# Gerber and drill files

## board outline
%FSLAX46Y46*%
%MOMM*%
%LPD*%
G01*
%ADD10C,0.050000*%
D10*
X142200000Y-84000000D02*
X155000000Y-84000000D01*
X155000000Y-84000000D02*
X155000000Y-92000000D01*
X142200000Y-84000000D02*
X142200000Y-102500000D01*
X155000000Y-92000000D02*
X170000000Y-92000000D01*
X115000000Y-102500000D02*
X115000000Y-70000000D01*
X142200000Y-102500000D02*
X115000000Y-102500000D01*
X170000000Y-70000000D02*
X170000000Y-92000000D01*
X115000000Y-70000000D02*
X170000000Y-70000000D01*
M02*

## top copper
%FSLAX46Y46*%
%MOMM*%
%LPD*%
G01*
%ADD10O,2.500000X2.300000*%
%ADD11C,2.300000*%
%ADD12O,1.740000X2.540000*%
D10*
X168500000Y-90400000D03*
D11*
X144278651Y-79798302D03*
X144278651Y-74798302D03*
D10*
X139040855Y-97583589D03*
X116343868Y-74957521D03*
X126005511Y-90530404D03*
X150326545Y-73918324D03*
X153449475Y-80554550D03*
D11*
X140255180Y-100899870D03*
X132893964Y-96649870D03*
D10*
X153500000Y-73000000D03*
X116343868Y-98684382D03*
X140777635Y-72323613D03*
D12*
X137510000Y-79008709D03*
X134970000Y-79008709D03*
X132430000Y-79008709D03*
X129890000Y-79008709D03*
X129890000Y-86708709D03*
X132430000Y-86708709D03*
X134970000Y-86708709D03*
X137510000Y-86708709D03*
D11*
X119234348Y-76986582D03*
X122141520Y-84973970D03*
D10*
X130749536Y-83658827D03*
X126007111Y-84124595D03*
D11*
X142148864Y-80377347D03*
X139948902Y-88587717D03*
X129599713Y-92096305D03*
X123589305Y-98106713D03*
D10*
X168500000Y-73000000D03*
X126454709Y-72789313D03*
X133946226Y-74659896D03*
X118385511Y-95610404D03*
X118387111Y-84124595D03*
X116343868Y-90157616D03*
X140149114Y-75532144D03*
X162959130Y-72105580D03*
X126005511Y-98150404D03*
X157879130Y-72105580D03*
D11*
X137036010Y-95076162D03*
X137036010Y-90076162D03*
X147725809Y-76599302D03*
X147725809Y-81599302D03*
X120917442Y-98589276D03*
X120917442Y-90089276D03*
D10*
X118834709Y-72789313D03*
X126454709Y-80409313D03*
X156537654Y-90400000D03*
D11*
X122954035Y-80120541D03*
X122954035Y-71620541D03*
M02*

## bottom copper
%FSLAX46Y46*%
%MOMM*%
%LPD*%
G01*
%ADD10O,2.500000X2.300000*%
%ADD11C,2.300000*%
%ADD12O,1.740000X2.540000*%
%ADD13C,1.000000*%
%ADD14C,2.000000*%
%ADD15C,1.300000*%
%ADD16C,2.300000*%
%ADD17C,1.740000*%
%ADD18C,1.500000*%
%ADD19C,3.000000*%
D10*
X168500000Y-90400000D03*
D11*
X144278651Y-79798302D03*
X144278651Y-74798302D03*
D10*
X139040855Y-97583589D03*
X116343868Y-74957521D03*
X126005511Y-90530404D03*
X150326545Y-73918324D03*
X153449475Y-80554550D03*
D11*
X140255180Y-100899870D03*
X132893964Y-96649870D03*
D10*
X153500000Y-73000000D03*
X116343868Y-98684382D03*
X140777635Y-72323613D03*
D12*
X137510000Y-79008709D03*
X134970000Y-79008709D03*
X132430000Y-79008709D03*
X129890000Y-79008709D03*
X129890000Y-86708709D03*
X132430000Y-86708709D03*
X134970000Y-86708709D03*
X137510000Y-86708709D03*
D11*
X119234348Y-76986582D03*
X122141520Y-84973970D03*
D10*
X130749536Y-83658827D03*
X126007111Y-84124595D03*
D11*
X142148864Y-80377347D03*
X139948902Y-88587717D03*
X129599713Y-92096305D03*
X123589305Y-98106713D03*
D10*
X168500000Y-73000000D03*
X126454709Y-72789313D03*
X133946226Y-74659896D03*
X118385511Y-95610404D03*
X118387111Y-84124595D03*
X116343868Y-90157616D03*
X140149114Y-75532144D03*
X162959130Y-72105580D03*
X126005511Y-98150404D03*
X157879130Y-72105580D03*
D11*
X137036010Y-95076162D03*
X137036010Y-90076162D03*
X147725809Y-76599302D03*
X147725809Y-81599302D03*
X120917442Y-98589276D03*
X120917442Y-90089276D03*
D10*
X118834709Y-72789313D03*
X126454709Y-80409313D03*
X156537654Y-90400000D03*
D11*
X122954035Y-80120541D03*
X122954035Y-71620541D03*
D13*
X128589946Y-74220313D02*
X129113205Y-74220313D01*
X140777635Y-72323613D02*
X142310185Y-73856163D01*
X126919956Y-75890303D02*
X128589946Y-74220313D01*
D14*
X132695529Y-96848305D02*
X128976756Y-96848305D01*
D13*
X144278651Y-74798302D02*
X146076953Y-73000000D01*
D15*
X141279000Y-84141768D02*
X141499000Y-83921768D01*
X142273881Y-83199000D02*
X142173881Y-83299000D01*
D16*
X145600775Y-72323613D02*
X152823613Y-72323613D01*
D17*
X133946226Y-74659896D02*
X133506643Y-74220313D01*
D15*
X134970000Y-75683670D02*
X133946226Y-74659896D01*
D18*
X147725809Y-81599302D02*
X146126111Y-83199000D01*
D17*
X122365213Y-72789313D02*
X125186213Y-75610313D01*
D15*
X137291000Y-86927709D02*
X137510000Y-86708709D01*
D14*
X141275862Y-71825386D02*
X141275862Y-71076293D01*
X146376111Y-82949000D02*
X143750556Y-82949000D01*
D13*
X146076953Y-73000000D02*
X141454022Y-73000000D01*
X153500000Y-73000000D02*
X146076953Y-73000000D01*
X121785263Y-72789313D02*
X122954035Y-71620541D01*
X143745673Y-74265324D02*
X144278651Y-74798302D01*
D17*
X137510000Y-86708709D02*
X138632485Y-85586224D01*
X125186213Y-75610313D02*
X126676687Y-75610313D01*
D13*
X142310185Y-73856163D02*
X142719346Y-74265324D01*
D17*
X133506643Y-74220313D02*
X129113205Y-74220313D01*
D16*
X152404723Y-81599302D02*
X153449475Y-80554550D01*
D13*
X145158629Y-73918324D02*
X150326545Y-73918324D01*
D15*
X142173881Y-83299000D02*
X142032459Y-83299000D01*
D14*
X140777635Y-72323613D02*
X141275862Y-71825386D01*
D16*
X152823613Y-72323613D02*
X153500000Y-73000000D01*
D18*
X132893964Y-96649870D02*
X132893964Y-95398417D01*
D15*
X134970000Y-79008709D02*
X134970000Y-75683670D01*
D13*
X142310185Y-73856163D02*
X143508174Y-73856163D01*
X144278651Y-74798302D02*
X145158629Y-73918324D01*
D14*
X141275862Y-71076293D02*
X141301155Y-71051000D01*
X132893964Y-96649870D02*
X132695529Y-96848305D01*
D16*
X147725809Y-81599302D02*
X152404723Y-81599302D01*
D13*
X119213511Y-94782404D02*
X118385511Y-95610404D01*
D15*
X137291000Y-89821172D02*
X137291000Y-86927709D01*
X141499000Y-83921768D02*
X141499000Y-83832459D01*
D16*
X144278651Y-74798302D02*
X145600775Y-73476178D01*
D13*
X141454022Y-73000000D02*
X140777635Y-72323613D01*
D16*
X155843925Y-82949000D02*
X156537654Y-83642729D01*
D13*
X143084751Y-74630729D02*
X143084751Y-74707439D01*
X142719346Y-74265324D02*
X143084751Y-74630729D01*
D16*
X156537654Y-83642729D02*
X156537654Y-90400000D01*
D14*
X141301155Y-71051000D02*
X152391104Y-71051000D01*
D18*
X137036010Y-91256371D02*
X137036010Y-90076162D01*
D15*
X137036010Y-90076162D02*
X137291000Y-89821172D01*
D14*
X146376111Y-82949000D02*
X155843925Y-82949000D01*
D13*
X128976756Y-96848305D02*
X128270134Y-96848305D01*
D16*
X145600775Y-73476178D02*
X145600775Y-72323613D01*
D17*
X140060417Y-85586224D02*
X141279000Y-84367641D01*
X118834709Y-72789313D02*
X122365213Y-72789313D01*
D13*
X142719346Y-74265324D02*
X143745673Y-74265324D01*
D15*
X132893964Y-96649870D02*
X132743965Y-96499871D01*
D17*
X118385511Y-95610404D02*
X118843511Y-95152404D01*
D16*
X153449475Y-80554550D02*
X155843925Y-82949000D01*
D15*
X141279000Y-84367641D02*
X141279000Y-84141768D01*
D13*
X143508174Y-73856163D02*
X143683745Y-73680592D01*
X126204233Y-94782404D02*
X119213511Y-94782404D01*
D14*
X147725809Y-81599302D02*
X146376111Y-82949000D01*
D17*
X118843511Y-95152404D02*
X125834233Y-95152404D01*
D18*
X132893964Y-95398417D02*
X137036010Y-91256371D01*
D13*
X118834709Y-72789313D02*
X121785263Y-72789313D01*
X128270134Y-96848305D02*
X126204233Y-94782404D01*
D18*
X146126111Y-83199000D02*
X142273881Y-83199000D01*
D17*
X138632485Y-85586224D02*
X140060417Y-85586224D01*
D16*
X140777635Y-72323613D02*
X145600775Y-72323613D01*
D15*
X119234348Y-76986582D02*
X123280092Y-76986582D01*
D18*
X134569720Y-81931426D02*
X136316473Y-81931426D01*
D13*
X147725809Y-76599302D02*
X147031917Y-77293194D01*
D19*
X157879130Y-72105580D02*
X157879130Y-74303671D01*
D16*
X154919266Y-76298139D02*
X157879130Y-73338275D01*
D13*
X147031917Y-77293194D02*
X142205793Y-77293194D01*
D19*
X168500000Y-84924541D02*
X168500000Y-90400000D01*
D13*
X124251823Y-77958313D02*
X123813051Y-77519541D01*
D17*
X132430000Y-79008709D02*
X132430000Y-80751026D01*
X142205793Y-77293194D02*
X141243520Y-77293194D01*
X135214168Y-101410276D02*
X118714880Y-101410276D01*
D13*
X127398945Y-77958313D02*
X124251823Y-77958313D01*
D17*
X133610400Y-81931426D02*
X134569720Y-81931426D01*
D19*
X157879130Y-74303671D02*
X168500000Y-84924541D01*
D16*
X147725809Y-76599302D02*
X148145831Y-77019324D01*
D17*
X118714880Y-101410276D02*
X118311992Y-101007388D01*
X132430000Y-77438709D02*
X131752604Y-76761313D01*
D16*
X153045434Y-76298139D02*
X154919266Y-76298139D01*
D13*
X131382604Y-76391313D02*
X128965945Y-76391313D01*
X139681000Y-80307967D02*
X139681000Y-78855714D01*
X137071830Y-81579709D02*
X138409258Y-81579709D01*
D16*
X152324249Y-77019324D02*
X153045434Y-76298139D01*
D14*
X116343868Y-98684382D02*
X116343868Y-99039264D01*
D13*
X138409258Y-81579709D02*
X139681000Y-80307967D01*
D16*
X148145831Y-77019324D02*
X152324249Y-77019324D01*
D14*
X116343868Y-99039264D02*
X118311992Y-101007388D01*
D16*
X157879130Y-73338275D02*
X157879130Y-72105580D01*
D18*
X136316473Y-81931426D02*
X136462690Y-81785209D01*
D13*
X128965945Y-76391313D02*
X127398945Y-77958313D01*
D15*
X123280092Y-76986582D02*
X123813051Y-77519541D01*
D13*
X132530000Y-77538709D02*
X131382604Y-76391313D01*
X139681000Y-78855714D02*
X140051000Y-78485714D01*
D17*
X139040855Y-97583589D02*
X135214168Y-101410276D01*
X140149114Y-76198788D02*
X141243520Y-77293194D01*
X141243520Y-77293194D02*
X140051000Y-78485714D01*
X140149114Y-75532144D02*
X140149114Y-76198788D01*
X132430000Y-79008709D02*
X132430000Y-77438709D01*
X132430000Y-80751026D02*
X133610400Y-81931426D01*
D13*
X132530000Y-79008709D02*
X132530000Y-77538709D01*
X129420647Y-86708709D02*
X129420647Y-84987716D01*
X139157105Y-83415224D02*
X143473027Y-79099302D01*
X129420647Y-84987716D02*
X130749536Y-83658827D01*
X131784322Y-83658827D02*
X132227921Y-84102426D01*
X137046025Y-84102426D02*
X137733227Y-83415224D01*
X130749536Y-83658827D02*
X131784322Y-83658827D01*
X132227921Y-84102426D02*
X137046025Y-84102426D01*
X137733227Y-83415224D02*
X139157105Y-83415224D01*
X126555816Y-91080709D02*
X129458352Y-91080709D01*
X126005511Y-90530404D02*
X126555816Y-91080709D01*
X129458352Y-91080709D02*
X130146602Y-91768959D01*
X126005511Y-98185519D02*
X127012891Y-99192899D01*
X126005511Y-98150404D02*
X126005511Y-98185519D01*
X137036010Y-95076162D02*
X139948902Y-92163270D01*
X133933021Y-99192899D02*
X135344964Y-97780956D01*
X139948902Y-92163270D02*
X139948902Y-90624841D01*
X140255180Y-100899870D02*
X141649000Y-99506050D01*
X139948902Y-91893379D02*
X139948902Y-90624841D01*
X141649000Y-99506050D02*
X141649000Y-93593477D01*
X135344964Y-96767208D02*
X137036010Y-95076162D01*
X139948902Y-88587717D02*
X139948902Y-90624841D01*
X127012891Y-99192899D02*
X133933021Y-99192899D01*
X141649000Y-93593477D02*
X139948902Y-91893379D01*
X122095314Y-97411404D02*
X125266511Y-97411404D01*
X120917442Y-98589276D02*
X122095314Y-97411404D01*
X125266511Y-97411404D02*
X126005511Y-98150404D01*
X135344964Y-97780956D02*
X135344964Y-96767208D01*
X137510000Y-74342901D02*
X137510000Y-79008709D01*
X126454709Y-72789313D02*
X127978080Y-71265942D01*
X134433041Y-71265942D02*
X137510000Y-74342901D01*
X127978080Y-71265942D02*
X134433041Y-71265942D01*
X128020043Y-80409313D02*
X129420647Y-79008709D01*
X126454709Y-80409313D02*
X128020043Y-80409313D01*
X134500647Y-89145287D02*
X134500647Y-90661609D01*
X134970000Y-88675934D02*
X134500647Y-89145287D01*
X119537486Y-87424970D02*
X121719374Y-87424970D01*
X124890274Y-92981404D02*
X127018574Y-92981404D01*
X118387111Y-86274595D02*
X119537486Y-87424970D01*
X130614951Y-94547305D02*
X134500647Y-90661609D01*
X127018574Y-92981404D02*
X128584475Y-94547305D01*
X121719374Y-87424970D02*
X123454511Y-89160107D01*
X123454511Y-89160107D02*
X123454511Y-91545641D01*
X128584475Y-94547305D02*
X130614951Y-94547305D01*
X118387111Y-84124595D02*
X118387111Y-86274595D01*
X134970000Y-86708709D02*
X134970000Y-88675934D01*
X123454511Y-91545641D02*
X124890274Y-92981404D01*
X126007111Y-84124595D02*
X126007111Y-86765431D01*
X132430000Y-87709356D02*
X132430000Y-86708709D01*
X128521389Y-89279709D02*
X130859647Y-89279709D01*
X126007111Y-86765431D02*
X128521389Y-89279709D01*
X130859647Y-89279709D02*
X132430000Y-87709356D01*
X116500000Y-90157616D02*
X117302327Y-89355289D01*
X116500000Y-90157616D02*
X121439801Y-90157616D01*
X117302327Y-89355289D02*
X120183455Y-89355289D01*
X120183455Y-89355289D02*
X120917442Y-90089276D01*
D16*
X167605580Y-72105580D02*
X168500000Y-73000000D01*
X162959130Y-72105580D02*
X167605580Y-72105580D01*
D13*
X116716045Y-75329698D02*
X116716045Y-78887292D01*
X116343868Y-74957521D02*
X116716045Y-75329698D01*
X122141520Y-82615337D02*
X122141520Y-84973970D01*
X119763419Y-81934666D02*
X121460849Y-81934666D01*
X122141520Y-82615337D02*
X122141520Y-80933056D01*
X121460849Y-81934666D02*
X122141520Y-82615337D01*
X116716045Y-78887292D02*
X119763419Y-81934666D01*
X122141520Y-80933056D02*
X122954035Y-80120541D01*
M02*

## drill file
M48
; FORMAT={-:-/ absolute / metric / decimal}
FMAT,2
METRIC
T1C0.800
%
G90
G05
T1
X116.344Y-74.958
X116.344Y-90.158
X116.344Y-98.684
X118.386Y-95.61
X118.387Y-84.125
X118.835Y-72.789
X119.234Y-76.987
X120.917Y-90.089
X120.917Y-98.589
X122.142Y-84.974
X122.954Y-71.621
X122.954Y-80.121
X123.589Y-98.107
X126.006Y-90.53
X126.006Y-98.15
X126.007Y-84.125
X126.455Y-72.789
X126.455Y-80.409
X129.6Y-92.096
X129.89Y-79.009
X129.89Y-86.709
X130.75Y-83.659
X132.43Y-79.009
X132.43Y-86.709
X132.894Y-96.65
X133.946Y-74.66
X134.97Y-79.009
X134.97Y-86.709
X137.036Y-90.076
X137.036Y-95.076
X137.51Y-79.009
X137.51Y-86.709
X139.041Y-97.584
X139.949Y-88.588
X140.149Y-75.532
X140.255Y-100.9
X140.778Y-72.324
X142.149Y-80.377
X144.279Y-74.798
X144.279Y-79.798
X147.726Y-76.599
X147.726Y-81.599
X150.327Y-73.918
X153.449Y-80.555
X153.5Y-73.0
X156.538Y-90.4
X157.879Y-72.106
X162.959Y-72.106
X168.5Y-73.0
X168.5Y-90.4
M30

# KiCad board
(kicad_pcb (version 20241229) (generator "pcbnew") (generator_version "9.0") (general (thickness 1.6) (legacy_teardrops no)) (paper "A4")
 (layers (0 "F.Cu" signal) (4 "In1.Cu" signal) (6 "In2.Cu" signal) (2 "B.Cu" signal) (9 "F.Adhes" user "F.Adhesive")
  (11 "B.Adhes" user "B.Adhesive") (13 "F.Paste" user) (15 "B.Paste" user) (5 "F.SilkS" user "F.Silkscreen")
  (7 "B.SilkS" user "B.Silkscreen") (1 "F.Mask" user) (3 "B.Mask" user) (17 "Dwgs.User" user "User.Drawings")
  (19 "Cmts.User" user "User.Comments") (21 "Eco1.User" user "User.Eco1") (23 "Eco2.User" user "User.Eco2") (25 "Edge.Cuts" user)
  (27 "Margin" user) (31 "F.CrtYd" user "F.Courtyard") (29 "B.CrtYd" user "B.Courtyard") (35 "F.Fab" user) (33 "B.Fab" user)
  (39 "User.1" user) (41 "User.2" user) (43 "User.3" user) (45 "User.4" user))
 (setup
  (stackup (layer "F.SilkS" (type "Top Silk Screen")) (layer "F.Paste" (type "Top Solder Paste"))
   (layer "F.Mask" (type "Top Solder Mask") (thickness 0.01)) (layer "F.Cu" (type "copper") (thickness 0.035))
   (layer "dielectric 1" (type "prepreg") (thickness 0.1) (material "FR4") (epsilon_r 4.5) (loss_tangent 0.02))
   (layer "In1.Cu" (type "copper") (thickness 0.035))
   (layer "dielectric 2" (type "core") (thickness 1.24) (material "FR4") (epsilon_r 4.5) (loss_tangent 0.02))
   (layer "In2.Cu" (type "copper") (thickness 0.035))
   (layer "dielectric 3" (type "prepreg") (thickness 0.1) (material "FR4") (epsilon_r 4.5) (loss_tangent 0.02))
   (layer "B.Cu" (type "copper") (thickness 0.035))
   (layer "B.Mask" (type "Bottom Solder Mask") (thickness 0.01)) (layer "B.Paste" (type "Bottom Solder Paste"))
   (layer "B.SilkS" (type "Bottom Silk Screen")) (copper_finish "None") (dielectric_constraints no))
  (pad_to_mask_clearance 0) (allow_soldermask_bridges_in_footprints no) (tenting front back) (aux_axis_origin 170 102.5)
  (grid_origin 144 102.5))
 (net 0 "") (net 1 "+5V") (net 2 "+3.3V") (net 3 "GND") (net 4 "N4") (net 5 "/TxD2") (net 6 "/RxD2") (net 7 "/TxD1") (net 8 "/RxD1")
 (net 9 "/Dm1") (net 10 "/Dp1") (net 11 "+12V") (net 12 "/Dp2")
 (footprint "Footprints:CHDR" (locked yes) (layer "F.Cu") (at 168.5 90.4)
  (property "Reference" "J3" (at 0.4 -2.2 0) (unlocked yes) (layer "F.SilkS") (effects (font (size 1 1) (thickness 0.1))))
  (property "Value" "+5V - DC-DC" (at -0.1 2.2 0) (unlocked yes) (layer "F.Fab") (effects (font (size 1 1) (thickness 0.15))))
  (pad "1" thru_hole oval (at 0 0) (size 2.5 2.3) (drill 0.8) (layers "*.Cu" "*.Mask") (remove_unused_layers no) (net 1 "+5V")))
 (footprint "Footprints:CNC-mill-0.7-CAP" (layer "F.Cu") (at 144.278651 77.298302)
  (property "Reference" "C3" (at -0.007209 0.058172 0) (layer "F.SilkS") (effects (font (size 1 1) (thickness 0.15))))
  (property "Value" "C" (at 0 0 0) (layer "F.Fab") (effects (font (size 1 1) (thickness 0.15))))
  (pad "1" thru_hole circle (at 0 2.5) (size 2.3 2.3) (drill 0.8) (layers "*.Cu" "*.Mask") (remove_unused_layers no) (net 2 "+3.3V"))
  (pad "2" thru_hole circle (at 0 -2.5) (size 2.3 2.3) (drill 0.8) (layers "*.Cu" "*.Mask") (remove_unused_layers no) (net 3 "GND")))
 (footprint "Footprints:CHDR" (layer "F.Cu") (at 139.040855 97.583589)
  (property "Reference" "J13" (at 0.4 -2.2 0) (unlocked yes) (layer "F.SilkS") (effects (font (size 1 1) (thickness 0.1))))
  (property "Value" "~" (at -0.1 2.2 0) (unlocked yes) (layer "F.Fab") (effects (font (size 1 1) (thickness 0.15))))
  (pad "1" thru_hole oval (at 0 0) (size 2.5 2.3) (drill 0.8) (layers "*.Cu" "*.Mask") (remove_unused_layers no) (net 1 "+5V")))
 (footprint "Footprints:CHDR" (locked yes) (layer "F.Cu") (at 116.343868 74.957521)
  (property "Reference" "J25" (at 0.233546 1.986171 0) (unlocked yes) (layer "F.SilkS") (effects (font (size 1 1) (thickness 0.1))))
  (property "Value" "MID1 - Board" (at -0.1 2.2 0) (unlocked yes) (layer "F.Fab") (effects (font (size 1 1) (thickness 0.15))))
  (pad "1" thru_hole oval (at 0 0) (size 2.5 2.3) (drill 0.8) (layers "*.Cu" "*.Mask") (remove_unused_layers no) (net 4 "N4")))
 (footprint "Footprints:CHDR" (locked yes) (layer "F.Cu") (at 126.005511 90.530404)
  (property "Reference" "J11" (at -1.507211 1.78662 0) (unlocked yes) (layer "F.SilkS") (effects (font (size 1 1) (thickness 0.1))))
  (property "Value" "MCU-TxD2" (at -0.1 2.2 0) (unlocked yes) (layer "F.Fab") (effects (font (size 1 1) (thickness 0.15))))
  (pad "1" thru_hole oval (at 0 0) (size 2.5 2.3) (drill 0.8) (layers "*.Cu" "*.Mask") (remove_unused_layers no) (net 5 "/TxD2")))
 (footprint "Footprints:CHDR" (layer "F.Cu") (at 150.326545 73.918324)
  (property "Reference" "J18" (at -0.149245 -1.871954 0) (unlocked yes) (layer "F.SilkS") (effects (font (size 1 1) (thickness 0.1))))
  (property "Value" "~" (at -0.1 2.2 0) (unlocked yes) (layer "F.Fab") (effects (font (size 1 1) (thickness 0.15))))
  (pad "1" thru_hole oval (at 0 0) (size 2.5 2.3) (drill 0.8) (layers "*.Cu" "*.Mask") (remove_unused_layers no) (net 3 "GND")))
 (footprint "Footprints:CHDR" (layer "F.Cu") (at 153.449475 80.55455)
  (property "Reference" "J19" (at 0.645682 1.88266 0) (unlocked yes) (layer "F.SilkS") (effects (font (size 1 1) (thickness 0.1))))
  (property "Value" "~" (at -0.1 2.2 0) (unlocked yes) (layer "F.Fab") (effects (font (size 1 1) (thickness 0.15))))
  (pad "1" thru_hole oval (at 0 0) (size 2.5 2.3) (drill 0.8) (layers "*.Cu" "*.Mask") (remove_unused_layers no) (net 3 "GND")))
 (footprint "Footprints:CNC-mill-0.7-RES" (layer "F.Cu") (at 136.574572 98.77487 60)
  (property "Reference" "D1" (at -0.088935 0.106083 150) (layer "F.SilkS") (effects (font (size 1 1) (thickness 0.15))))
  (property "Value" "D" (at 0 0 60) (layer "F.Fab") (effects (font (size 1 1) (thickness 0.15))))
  (pad "1" thru_hole circle (at 0 4.25 60) (size 2.3 2.3) (drill 0.8) (layers "*.Cu" "*.Mask") (remove_unused_layers no) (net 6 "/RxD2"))
  (pad "2" thru_hole circle (at 0 -4.25 60) (size 2.3 2.3) (drill 0.8) (layers "*.Cu" "*.Mask") (remove_unused_layers no) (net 3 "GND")))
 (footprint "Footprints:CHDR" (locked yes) (layer "F.Cu") (at 153.5 73)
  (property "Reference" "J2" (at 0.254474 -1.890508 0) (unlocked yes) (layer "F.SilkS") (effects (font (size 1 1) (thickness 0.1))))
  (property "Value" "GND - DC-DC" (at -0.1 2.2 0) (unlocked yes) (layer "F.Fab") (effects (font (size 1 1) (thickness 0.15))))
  (pad "1" thru_hole oval (at 0 0) (size 2.5 2.3) (drill 0.8) (layers "*.Cu" "*.Mask") (remove_unused_layers no) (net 3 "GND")))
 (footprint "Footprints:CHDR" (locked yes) (layer "F.Cu") (at 116.343868 98.684382)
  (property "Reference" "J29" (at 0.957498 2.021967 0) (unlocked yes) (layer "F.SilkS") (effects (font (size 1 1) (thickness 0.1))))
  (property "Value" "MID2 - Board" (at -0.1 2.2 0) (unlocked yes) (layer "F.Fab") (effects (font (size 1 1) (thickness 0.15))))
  (pad "1" thru_hole oval (at 0 0) (size 2.5 2.3) (drill 0.8) (layers "*.Cu" "*.Mask") (remove_unused_layers no) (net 1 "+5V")))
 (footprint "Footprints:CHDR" (layer "F.Cu") (at 140.777635 72.323613)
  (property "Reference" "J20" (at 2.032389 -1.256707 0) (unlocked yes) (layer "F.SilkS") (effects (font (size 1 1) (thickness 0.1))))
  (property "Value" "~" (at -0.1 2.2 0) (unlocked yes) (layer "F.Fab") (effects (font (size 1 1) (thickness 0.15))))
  (pad "1" thru_hole oval (at 0 0) (size 2.5 2.3) (drill 0.8) (layers "*.Cu" "*.Mask") (remove_unused_layers no) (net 3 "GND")))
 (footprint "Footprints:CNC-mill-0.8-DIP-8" (layer "F.Cu") (at 133.7 82.858709 180)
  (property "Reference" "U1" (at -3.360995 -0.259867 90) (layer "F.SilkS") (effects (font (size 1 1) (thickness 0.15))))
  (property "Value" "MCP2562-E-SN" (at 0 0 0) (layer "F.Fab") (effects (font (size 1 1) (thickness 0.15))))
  (pad "1" thru_hole oval (at -3.81 3.85 180) (size 1.74 2.54) (drill 0.8) (layers "*.Cu" "*.Mask") (remove_unused_layers no)
   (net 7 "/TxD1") (thermal_bridge_angle 45))
  (pad "2" thru_hole oval (at -1.27 3.85 180) (size 1.74 2.54) (drill 0.8) (layers "*.Cu" "*.Mask") (remove_unused_layers no) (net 3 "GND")
   (thermal_bridge_angle 45))
  (pad "3" thru_hole oval (at 1.27 3.85 180) (size 1.74 2.54) (drill 0.8) (layers "*.Cu" "*.Mask") (remove_unused_layers no) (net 1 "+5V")
   (thermal_bridge_angle 45))
  (pad "4" thru_hole oval (at 3.81 3.85 180) (size 1.74 2.54) (drill 0.8) (layers "*.Cu" "*.Mask") (remove_unused_layers no) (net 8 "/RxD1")
   (thermal_bridge_angle 45))
  (pad "5" thru_hole oval (at 3.81 -3.85 180) (size 1.74 2.54) (drill 0.8) (layers "*.Cu" "*.Mask") (remove_unused_layers no)
   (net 2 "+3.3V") (thermal_bridge_angle 45))
  (pad "6" thru_hole oval (at 1.27 -3.85 180) (size 1.74 2.54) (drill 0.8) (layers "*.Cu" "*.Mask") (remove_unused_layers no) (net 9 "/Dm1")
   (thermal_bridge_angle 45))
  (pad "7" thru_hole oval (at -1.27 -3.85 180) (size 1.74 2.54) (drill 0.8) (layers "*.Cu" "*.Mask") (remove_unused_layers no)
   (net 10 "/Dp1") (thermal_bridge_angle 45))
  (pad "8" thru_hole oval (at -3.81 -3.85 180) (size 1.74 2.54) (drill 0.8) (layers "*.Cu" "*.Mask") (remove_unused_layers no) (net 3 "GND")
   (thermal_bridge_angle 45)))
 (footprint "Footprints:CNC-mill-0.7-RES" (layer "F.Cu") (at 120.687934 80.980276 -160)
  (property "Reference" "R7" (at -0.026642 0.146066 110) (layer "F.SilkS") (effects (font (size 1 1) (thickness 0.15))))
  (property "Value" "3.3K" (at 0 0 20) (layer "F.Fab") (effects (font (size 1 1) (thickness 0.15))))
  (pad "1" thru_hole circle (at 0 4.25 200) (size 2.3 2.3) (drill 0.8) (layers "*.Cu" "*.Mask") (remove_unused_layers no) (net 1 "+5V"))
  (pad "2" thru_hole circle (at 0 -4.25 200) (size 2.3 2.3) (drill 0.8) (layers "*.Cu" "*.Mask") (remove_unused_layers no) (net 4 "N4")))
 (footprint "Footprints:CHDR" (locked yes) (layer "F.Cu") (at 130.749536 83.658827)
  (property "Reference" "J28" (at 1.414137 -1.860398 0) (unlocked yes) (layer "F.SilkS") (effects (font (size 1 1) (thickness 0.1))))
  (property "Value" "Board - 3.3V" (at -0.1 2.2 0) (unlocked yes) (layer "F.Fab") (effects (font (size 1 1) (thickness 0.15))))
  (pad "1" thru_hole oval (at 0 0) (size 2.5 2.3) (drill 0.8) (layers "*.Cu" "*.Mask") (remove_unused_layers no) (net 2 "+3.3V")))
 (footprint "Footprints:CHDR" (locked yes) (layer "F.Cu") (at 126.007111 84.124595)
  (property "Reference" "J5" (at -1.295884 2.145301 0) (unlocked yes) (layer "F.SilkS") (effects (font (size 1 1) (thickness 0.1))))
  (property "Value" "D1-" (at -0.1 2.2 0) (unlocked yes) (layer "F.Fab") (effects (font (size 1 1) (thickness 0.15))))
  (pad "1" thru_hole oval (at 0 0) (size 2.5 2.3) (drill 0.8) (layers "*.Cu" "*.Mask") (remove_unused_layers no) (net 9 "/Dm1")))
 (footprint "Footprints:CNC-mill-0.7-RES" (layer "F.Cu") (at 141.048883 84.482532 165)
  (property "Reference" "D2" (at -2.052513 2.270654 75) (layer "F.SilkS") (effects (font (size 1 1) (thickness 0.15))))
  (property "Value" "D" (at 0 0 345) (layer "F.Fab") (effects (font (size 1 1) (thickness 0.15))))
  (pad "1" thru_hole circle (at 0 4.25 165) (size 2.3 2.3) (drill 0.8) (layers "*.Cu" "*.Mask") (remove_unused_layers no) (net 2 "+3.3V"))
  (pad "2" thru_hole circle (at 0 -4.25 165) (size 2.3 2.3) (drill 0.8) (layers "*.Cu" "*.Mask") (remove_unused_layers no) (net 6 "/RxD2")))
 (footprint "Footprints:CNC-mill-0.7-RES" (layer "F.Cu") (at 126.594509 95.101509 135)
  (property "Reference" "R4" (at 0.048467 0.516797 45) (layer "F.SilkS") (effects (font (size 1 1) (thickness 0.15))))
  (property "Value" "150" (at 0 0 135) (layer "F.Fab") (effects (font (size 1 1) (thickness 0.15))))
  (pad "1" thru_hole circle (at 0 4.25 135) (size 2.3 2.3) (drill 0.8) (layers "*.Cu" "*.Mask") (remove_unused_layers no) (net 5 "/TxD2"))
  (pad "2" thru_hole circle (at 0 -4.25 135) (size 2.3 2.3) (drill 0.8) (layers "*.Cu" "*.Mask") (remove_unused_layers no) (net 6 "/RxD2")))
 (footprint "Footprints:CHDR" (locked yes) (layer "F.Cu") (at 168.5 73)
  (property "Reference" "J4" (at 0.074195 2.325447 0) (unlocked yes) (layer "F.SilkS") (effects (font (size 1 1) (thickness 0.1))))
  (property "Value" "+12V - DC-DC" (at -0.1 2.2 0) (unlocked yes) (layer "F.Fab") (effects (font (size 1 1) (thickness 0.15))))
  (pad "1" thru_hole oval (at 0 0) (size 2.5 2.3) (drill 0.8) (layers "*.Cu" "*.Mask") (remove_unused_layers no) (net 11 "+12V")))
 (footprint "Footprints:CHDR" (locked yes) (layer "F.Cu") (at 126.454709 72.789313)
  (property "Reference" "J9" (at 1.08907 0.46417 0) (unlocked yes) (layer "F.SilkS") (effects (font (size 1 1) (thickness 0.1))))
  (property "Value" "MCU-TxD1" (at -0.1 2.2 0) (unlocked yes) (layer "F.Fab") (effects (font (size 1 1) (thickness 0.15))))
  (pad "1" thru_hole oval (at 0 0) (size 2.5 2.3) (drill 0.8) (layers "*.Cu" "*.Mask") (remove_unused_layers no) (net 7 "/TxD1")))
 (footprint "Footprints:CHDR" (layer "F.Cu") (at 133.946226 74.659896)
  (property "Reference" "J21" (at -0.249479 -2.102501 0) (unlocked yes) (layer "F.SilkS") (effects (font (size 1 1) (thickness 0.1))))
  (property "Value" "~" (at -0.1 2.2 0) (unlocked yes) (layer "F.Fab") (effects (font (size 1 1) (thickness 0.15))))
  (pad "1" thru_hole oval (at 0 0) (size 2.5 2.3) (drill 0.8) (layers "*.Cu" "*.Mask") (remove_unused_layers no) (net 3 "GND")))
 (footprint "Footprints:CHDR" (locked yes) (layer "F.Cu") (at 118.385511 95.610404)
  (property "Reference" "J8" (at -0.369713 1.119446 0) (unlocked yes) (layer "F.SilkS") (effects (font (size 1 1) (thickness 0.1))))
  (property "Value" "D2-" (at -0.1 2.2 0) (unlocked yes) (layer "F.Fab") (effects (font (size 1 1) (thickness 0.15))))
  (pad "1" thru_hole oval (at 0 0) (size 2.5 2.3) (drill 0.8) (layers "*.Cu" "*.Mask") (remove_unused_layers no) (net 3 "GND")))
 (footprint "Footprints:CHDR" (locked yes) (layer "F.Cu") (at 118.387111 84.124595)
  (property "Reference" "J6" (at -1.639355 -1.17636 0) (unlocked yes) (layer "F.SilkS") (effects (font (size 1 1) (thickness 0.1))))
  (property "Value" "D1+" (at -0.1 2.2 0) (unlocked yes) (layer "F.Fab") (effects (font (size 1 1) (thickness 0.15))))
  (pad "1" thru_hole oval (at 0 0) (size 2.5 2.3) (drill 0.8) (layers "*.Cu" "*.Mask") (remove_unused_layers no) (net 10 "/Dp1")))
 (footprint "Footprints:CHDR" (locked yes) (layer "F.Cu") (at 116.343868 90.157616)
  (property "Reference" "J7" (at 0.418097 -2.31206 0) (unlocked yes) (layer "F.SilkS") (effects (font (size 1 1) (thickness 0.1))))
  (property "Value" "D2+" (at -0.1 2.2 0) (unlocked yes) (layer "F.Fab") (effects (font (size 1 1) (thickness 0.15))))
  (pad "1" thru_hole oval (at 0 0) (size 2.5 2.3) (drill 0.8) (layers "*.Cu" "*.Mask") (remove_unused_layers no) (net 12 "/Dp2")))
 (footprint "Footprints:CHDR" (layer "F.Cu") (at 140.149114 75.532144)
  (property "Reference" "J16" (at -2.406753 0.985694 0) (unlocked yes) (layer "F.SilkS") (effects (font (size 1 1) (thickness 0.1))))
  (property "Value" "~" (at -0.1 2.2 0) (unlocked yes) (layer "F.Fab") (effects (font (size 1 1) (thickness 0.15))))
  (pad "1" thru_hole oval (at 0 0) (size 2.5 2.3) (drill 0.8) (layers "*.Cu" "*.Mask") (remove_unused_layers no) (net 1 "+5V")))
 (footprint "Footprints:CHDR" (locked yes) (layer "F.Cu") (at 162.95913 72.10558)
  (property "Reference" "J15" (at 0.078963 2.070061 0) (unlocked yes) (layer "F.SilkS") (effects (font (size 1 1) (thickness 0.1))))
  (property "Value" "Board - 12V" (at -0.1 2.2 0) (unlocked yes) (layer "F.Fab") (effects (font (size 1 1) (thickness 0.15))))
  (pad "1" thru_hole oval (at 0 0) (size 2.5 2.3) (drill 0.8) (layers "*.Cu" "*.Mask") (remove_unused_layers no) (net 11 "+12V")))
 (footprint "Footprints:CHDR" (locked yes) (layer "F.Cu") (at 126.005511 98.150404)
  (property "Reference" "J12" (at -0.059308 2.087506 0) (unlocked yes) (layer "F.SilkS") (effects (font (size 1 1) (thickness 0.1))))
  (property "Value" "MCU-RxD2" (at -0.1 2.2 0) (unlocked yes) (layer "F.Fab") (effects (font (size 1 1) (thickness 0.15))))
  (pad "1" thru_hole oval (at 0 0) (size 2.5 2.3) (drill 0.8) (layers "*.Cu" "*.Mask") (remove_unused_layers no) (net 6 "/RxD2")))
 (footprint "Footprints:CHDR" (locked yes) (layer "F.Cu") (at 157.87913 72.10558)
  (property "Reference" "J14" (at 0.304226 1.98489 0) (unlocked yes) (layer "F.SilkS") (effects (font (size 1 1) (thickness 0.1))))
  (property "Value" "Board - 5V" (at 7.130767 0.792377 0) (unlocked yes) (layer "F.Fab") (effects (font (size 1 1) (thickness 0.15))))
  (pad "1" thru_hole oval (at 0 0) (size 2.5 2.3) (drill 0.8) (layers "*.Cu" "*.Mask") (remove_unused_layers no) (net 1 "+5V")))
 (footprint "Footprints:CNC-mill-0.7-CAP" (layer "F.Cu") (at 137.03601 92.576162)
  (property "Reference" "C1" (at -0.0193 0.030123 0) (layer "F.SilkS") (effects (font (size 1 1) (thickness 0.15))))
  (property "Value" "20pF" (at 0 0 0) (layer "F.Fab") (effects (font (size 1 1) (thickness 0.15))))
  (pad "1" thru_hole circle (at 0 2.5) (size 2.3 2.3) (drill 0.8) (layers "*.Cu" "*.Mask") (remove_unused_layers no) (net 6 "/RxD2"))
  (pad "2" thru_hole circle (at 0 -2.5) (size 2.3 2.3) (drill 0.8) (layers "*.Cu" "*.Mask") (remove_unused_layers no) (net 3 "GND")))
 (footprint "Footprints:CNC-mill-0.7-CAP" (layer "F.Cu") (at 147.725809 79.099302 180)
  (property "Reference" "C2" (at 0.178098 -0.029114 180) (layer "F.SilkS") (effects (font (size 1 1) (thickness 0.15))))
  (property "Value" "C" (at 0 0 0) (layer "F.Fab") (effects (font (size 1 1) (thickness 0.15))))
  (pad "1" thru_hole circle (at 0 2.5 180) (size 2.3 2.3) (drill 0.8) (layers "*.Cu" "*.Mask") (remove_unused_layers no) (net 1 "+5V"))
  (pad "2" thru_hole circle (at 0 -2.5 180) (size 2.3 2.3) (drill 0.8) (layers "*.Cu" "*.Mask") (remove_unused_layers no) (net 3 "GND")))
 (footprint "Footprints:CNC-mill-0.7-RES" (layer "F.Cu") (at 120.917442 94.339276)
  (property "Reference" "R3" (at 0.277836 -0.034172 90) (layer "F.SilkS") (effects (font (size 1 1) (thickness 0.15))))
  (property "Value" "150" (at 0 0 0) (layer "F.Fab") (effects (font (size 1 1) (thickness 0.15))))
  (pad "1" thru_hole circle (at 0 4.25) (size 2.3 2.3) (drill 0.8) (layers "*.Cu" "*.Mask") (remove_unused_layers no) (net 6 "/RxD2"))
  (pad "2" thru_hole circle (at 0 -4.25) (size 2.3 2.3) (drill 0.8) (layers "*.Cu" "*.Mask") (remove_unused_layers no) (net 12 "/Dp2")))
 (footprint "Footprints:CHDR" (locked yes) (layer "F.Cu") (at 118.834709 72.789313)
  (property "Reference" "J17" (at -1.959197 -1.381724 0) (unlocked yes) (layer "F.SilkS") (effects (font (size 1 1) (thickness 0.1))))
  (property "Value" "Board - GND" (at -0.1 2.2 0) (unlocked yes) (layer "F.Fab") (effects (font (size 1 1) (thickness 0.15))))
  (pad "1" thru_hole oval (at 0 0) (size 2.5 2.3) (drill 0.8) (layers "*.Cu" "*.Mask") (remove_unused_layers no) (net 3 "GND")))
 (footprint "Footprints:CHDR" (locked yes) (layer "F.Cu") (at 126.454709 80.409313)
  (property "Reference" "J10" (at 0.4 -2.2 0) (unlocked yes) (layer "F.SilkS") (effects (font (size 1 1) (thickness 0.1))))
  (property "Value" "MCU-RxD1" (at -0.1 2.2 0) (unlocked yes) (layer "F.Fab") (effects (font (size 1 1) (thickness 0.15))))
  (pad "1" thru_hole oval (at 0 0) (size 2.5 2.3) (drill 0.8) (layers "*.Cu" "*.Mask") (remove_unused_layers no) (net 8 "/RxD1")))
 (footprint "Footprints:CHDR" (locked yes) (layer "F.Cu") (at 156.537654 90.4)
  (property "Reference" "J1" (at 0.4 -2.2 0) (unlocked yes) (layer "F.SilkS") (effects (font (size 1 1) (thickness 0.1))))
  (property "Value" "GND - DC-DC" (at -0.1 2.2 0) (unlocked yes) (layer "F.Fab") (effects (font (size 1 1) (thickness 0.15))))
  (pad "1" thru_hole oval (at 0 0) (size 2.5 2.3) (drill 0.8) (layers "*.Cu" "*.Mask") (remove_unused_layers no) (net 3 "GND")))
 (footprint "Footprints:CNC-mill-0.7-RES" (layer "F.Cu") (at 122.954035 75.870541)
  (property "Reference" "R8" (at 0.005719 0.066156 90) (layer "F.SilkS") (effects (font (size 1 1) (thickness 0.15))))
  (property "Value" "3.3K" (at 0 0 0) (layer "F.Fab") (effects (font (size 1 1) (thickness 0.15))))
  (pad "1" thru_hole circle (at 0 4.25) (size 2.3 2.3) (drill 0.8) (layers "*.Cu" "*.Mask") (remove_unused_layers no) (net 4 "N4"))
  (pad "2" thru_hole circle (at 0 -4.25) (size 2.3 2.3) (drill 0.8) (layers "*.Cu" "*.Mask") (remove_unused_layers no) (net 3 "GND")))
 (gr_line (start 142.2 84) (end 155 84) (stroke (width 0.05) (type default)) (locked yes) (layer "Edge.Cuts"))
 (gr_line (start 155 84) (end 155 92) (stroke (width 0.05) (type default)) (locked yes) (layer "Edge.Cuts"))
 (gr_line (start 142.2 84) (end 142.2 102.5) (stroke (width 0.05) (type default)) (locked yes) (layer "Edge.Cuts"))
 (gr_line (start 155 92) (end 170 92) (stroke (width 0.05) (type default)) (locked yes) (layer "Edge.Cuts"))
 (gr_line (start 115 102.5) (end 115 70) (stroke (width 0.05) (type default)) (locked yes) (layer "Edge.Cuts"))
 (gr_line (start 142.2 102.5) (end 115 102.5) (stroke (width 0.05) (type default)) (locked yes) (layer "Edge.Cuts"))
 (gr_line (start 170 70) (end 170 92) (stroke (width 0.05) (type default)) (locked yes) (layer "Edge.Cuts"))
 (gr_line (start 115 70) (end 170 70) (stroke (width 0.05) (type default)) (locked yes) (layer "Edge.Cuts"))
 (segment (start 128.589946 74.220313) (end 129.113205 74.220313) (width 1) (layer "B.Cu") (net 3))
 (segment (start 140.777635 72.323613) (end 142.310185 73.856163) (width 1) (layer "B.Cu") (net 3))
 (segment (start 126.919956 75.890303) (end 128.589946 74.220313) (width 1) (layer "B.Cu") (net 3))
 (segment (start 132.695529 96.848305) (end 128.976756 96.848305) (width 2) (layer "B.Cu") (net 3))
 (segment (start 144.278651 74.798302) (end 146.076953 73) (width 1) (layer "B.Cu") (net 3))
 (segment (start 141.279 84.141768) (end 141.499 83.921768) (width 1.3) (layer "B.Cu") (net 3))
 (segment (start 142.273881 83.199) (end 142.173881 83.299) (width 1.3) (layer "B.Cu") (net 3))
 (segment (start 145.600775 72.323613) (end 152.823613 72.323613) (width 2.3) (layer "B.Cu") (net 3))
 (segment (start 133.946226 74.659896) (end 133.506643 74.220313) (width 1.74) (layer "B.Cu") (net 3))
 (segment (start 134.97 75.68367) (end 133.946226 74.659896) (width 1.3) (layer "B.Cu") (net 3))
 (segment (start 147.725809 81.599302) (end 146.126111 83.199) (width 1.5) (layer "B.Cu") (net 3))
 (segment (start 122.365213 72.789313) (end 125.186213 75.610313) (width 1.74) (layer "B.Cu") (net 3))
 (segment (start 137.291 86.927709) (end 137.51 86.708709) (width 1.3) (layer "B.Cu") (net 3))
 (segment (start 141.275862 71.825386) (end 141.275862 71.076293) (width 2) (layer "B.Cu") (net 3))
 (segment (start 146.376111 82.949) (end 143.750556 82.949) (width 2) (layer "B.Cu") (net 3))
 (segment (start 146.076953 73) (end 141.454022 73) (width 1) (layer "B.Cu") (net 3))
 (segment (start 153.5 73) (end 146.076953 73) (width 1) (layer "B.Cu") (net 3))
 (segment (start 121.785263 72.789313) (end 122.954035 71.620541) (width 1) (layer "B.Cu") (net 3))
 (segment (start 143.745673 74.265324) (end 144.278651 74.798302) (width 1) (layer "B.Cu") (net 3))
 (segment (start 137.51 86.708709) (end 138.632485 85.586224) (width 1.74) (layer "B.Cu") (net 3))
 (segment (start 125.186213 75.610313) (end 126.676687 75.610313) (width 1.74) (layer "B.Cu") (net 3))
 (segment (start 142.310185 73.856163) (end 142.719346 74.265324) (width 1) (layer "B.Cu") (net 3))
 (segment (start 133.506643 74.220313) (end 129.113205 74.220313) (width 1.74) (layer "B.Cu") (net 3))
 (segment (start 152.404723 81.599302) (end 153.449475 80.55455) (width 2.3) (layer "B.Cu") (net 3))
 (segment (start 145.158629 73.918324) (end 150.326545 73.918324) (width 1) (layer "B.Cu") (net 3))
 (segment (start 142.173881 83.299) (end 142.032459 83.299) (width 1.3) (layer "B.Cu") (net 3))
 (segment (start 140.777635 72.323613) (end 141.275862 71.825386) (width 2) (layer "B.Cu") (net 3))
 (segment (start 152.823613 72.323613) (end 153.5 73) (width 2.3) (layer "B.Cu") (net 3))
 (segment (start 132.893964 96.64987) (end 132.893964 95.398417) (width 1.5) (layer "B.Cu") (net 3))
 (segment (start 134.97 79.008709) (end 134.97 75.68367) (width 1.3) (layer "B.Cu") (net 3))
 (segment (start 142.310185 73.856163) (end 143.508174 73.856163) (width 1) (layer "B.Cu") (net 3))
 (segment (start 144.278651 74.798302) (end 145.158629 73.918324) (width 1) (layer "B.Cu") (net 3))
 (segment (start 141.275862 71.076293) (end 141.301155 71.051) (width 2) (layer "B.Cu") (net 3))
 (segment (start 132.893964 96.64987) (end 132.695529 96.848305) (width 2) (layer "B.Cu") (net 3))
 (segment (start 147.725809 81.599302) (end 152.404723 81.599302) (width 2.3) (layer "B.Cu") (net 3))
 (segment (start 119.213511 94.782404) (end 118.385511 95.610404) (width 1) (layer "B.Cu") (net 3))
 (segment (start 137.291 89.821172) (end 137.291 86.927709) (width 1.3) (layer "B.Cu") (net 3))
 (segment (start 141.499 83.921768) (end 141.499 83.832459) (width 1.3) (layer "B.Cu") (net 3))
 (segment (start 144.278651 74.798302) (end 145.600775 73.476178) (width 2.3) (layer "B.Cu") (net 3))
 (segment (start 141.454022 73) (end 140.777635 72.323613) (width 1) (layer "B.Cu") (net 3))
 (segment (start 155.843925 82.949) (end 156.537654 83.642729) (width 2.3) (layer "B.Cu") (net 3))
 (segment (start 143.084751 74.630729) (end 143.084751 74.707439) (width 1) (layer "B.Cu") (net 3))
 (segment (start 142.719346 74.265324) (end 143.084751 74.630729) (width 1) (layer "B.Cu") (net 3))
 (segment (start 156.537654 83.642729) (end 156.537654 90.4) (width 2.3) (layer "B.Cu") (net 3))
 (segment (start 141.301155 71.051) (end 152.391104 71.051) (width 2) (layer "B.Cu") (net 3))
 (segment (start 137.03601 91.256371) (end 137.03601 90.076162) (width 1.5) (layer "B.Cu") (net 3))
 (segment (start 137.03601 90.076162) (end 137.291 89.821172) (width 1.3) (layer "B.Cu") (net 3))
 (segment (start 146.376111 82.949) (end 155.843925 82.949) (width 2) (layer "B.Cu") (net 3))
 (segment (start 128.976756 96.848305) (end 128.270134 96.848305) (width 1) (layer "B.Cu") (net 3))
 (segment (start 145.600775 73.476178) (end 145.600775 72.323613) (width 2.3) (layer "B.Cu") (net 3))
 (segment (start 140.060417 85.586224) (end 141.279 84.367641) (width 1.74) (layer "B.Cu") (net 3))
 (segment (start 118.834709 72.789313) (end 122.365213 72.789313) (width 1.74) (layer "B.Cu") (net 3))
 (segment (start 142.719346 74.265324) (end 143.745673 74.265324) (width 1) (layer "B.Cu") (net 3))
 (segment (start 132.893964 96.64987) (end 132.743965 96.499871) (width 1.3) (layer "B.Cu") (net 3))
 (segment (start 118.385511 95.610404) (end 118.843511 95.152404) (width 1.74) (layer "B.Cu") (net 3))
 (segment (start 153.449475 80.55455) (end 155.843925 82.949) (width 2.3) (layer "B.Cu") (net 3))
 (segment (start 141.279 84.367641) (end 141.279 84.141768) (width 1.3) (layer "B.Cu") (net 3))
 (segment (start 143.508174 73.856163) (end 143.683745 73.680592) (width 1) (layer "B.Cu") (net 3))
 (segment (start 126.204233 94.782404) (end 119.213511 94.782404) (width 1) (layer "B.Cu") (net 3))
 (segment (start 147.725809 81.599302) (end 146.376111 82.949) (width 2) (layer "B.Cu") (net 3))
 (segment (start 118.843511 95.152404) (end 125.834233 95.152404) (width 1.74) (layer "B.Cu") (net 3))
 (segment (start 132.893964 95.398417) (end 137.03601 91.256371) (width 1.5) (layer "B.Cu") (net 3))
 (segment (start 118.834709 72.789313) (end 121.785263 72.789313) (width 1) (layer "B.Cu") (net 3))
 (segment (start 128.270134 96.848305) (end 126.204233 94.782404) (width 1) (layer "B.Cu") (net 3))
 (segment (start 146.126111 83.199) (end 142.273881 83.199) (width 1.5) (layer "B.Cu") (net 3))
 (segment (start 138.632485 85.586224) (end 140.060417 85.586224) (width 1.74) (layer "B.Cu") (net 3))
 (segment (start 140.777635 72.323613) (end 145.600775 72.323613) (width 2.3) (layer "B.Cu") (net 3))
 (segment (start 119.234348 76.986582) (end 123.280092 76.986582) (width 1.3) (layer "B.Cu") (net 1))
 (segment (start 134.56972 81.931426) (end 136.316473 81.931426) (width 1.5) (layer "B.Cu") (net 1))
 (segment (start 147.725809 76.599302) (end 147.031917 77.293194) (width 1) (layer "B.Cu") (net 1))
 (segment (start 157.87913 72.10558) (end 157.87913 74.303671) (width 3) (layer "B.Cu") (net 1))
 (segment (start 154.919266 76.298139) (end 157.87913 73.338275) (width 2.3) (layer "B.Cu") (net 1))
 (segment (start 147.031917 77.293194) (end 142.205793 77.293194) (width 1) (layer "B.Cu") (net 1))
 (segment (start 168.5 84.924541) (end 168.5 90.4) (width 3) (layer "B.Cu") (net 1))
 (segment (start 124.251823 77.958313) (end 123.813051 77.519541) (width 1) (layer "B.Cu") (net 1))
 (segment (start 132.43 79.008709) (end 132.43 80.751026) (width 1.74) (layer "B.Cu") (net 1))
 (segment (start 142.205793 77.293194) (end 141.24352 77.293194) (width 1.74) (layer "B.Cu") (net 1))
 (segment (start 135.214168 101.410276) (end 118.71488 101.410276) (width 1.74) (layer "B.Cu") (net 1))
 (segment (start 127.398945 77.958313) (end 124.251823 77.958313) (width 1) (layer "B.Cu") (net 1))
 (segment (start 133.6104 81.931426) (end 134.56972 81.931426) (width 1.74) (layer "B.Cu") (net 1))
 (segment (start 157.87913 74.303671) (end 168.5 84.924541) (width 3) (layer "B.Cu") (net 1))
 (segment (start 147.725809 76.599302) (end 148.145831 77.019324) (width 2.3) (layer "B.Cu") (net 1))
 (segment (start 118.71488 101.410276) (end 118.311992 101.007388) (width 1.74) (layer "B.Cu") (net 1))
 (segment (start 132.43 77.438709) (end 131.752604 76.761313) (width 1.74) (layer "B.Cu") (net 1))
 (segment (start 153.045434 76.298139) (end 154.919266 76.298139) (width 2.3) (layer "B.Cu") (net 1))
 (segment (start 131.382604 76.391313) (end 128.965945 76.391313) (width 1) (layer "B.Cu") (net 1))
 (segment (start 139.681 80.307967) (end 139.681 78.855714) (width 1) (layer "B.Cu") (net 1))
 (segment (start 137.07183 81.579709) (end 138.409258 81.579709) (width 1) (layer "B.Cu") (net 1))
 (segment (start 152.324249 77.019324) (end 153.045434 76.298139) (width 2.3) (layer "B.Cu") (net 1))
 (segment (start 116.343868 98.684382) (end 116.343868 99.039264) (width 2) (layer "B.Cu") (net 1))
 (segment (start 138.409258 81.579709) (end 139.681 80.307967) (width 1) (layer "B.Cu") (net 1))
 (segment (start 148.145831 77.019324) (end 152.324249 77.019324) (width 2.3) (layer "B.Cu") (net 1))
 (segment (start 116.343868 99.039264) (end 118.311992 101.007388) (width 2) (layer "B.Cu") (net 1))
 (segment (start 157.87913 73.338275) (end 157.87913 72.10558) (width 2.3) (layer "B.Cu") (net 1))
 (segment (start 136.316473 81.931426) (end 136.46269 81.785209) (width 1.5) (layer "B.Cu") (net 1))
 (segment (start 128.965945 76.391313) (end 127.398945 77.958313) (width 1) (layer "B.Cu") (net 1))
 (segment (start 123.280092 76.986582) (end 123.813051 77.519541) (width 1.3) (layer "B.Cu") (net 1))
 (segment (start 132.53 77.538709) (end 131.382604 76.391313) (width 1) (layer "B.Cu") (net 1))
 (segment (start 139.681 78.855714) (end 140.051 78.485714) (width 1) (layer "B.Cu") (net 1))
 (segment (start 139.040855 97.583589) (end 135.214168 101.410276) (width 1.74) (layer "B.Cu") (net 1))
 (segment (start 140.149114 76.198788) (end 141.24352 77.293194) (width 1.74) (layer "B.Cu") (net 1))
 (segment (start 141.24352 77.293194) (end 140.051 78.485714) (width 1.74) (layer "B.Cu") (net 1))
 (segment (start 140.149114 75.532144) (end 140.149114 76.198788) (width 1.74) (layer "B.Cu") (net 1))
 (segment (start 132.43 79.008709) (end 132.43 77.438709) (width 1.74) (layer "B.Cu") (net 1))
 (segment (start 132.43 80.751026) (end 133.6104 81.931426) (width 1.74) (layer "B.Cu") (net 1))
 (segment (start 132.53 79.008709) (end 132.53 77.538709) (width 1) (layer "B.Cu") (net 1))
 (segment (start 129.420647 86.708709) (end 129.420647 84.987716) (width 1) (layer "B.Cu") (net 2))
 (segment (start 139.157105 83.415224) (end 143.473027 79.099302) (width 1) (layer "B.Cu") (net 2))
 (segment (start 129.420647 84.987716) (end 130.749536 83.658827) (width 1) (layer "B.Cu") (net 2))
 (segment (start 131.784322 83.658827) (end 132.227921 84.102426) (width 1) (layer "B.Cu") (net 2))
 (segment (start 137.046025 84.102426) (end 137.733227 83.415224) (width 1) (layer "B.Cu") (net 2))
 (segment (start 130.749536 83.658827) (end 131.784322 83.658827) (width 1) (layer "B.Cu") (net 2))
 (segment (start 132.227921 84.102426) (end 137.046025 84.102426) (width 1) (layer "B.Cu") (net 2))
 (segment (start 137.733227 83.415224) (end 139.157105 83.415224) (width 1) (layer "B.Cu") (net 2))
 (segment (start 126.555816 91.080709) (end 129.458352 91.080709) (width 1) (layer "B.Cu") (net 5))
 (segment (start 126.005511 90.530404) (end 126.555816 91.080709) (width 1) (layer "B.Cu") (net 5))
 (segment (start 129.458352 91.080709) (end 130.146602 91.768959) (width 1) (layer "B.Cu") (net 5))
 (segment (start 126.005511 98.185519) (end 127.012891 99.192899) (width 1) (layer "B.Cu") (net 6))
 (segment (start 126.005511 98.150404) (end 126.005511 98.185519) (width 1) (layer "B.Cu") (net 6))
 (segment (start 137.03601 95.076162) (end 139.948902 92.16327) (width 1) (layer "B.Cu") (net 6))
 (segment (start 133.933021 99.192899) (end 135.344964 97.780956) (width 1) (layer "B.Cu") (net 6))
 (segment (start 139.948902 92.16327) (end 139.948902 90.624841) (width 1) (layer "B.Cu") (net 6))
 (segment (start 140.25518 100.89987) (end 141.649 99.50605) (width 1) (layer "B.Cu") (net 6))
 (segment (start 139.948902 91.893379) (end 139.948902 90.624841) (width 1) (layer "B.Cu") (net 6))
 (segment (start 141.649 99.50605) (end 141.649 93.593477) (width 1) (layer "B.Cu") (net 6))
 (segment (start 135.344964 96.767208) (end 137.03601 95.076162) (width 1) (layer "B.Cu") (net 6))
 (segment (start 139.948902 88.587717) (end 139.948902 90.624841) (width 1) (layer "B.Cu") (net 6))
 (segment (start 127.012891 99.192899) (end 133.933021 99.192899) (width 1) (layer "B.Cu") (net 6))
 (segment (start 141.649 93.593477) (end 139.948902 91.893379) (width 1) (layer "B.Cu") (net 6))
 (segment (start 122.095314 97.411404) (end 125.266511 97.411404) (width 1) (layer "B.Cu") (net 6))
 (segment (start 120.917442 98.589276) (end 122.095314 97.411404) (width 1) (layer "B.Cu") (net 6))
 (segment (start 125.266511 97.411404) (end 126.005511 98.150404) (width 1) (layer "B.Cu") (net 6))
 (segment (start 135.344964 97.780956) (end 135.344964 96.767208) (width 1) (layer "B.Cu") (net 6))
 (segment (start 137.51 74.342901) (end 137.51 79.008709) (width 1) (layer "B.Cu") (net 7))
 (segment (start 126.454709 72.789313) (end 127.97808 71.265942) (width 1) (layer "B.Cu") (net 7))
 (segment (start 134.433041 71.265942) (end 137.51 74.342901) (width 1) (layer "B.Cu") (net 7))
 (segment (start 127.97808 71.265942) (end 134.433041 71.265942) (width 1) (layer "B.Cu") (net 7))
 (segment (start 128.020043 80.409313) (end 129.420647 79.008709) (width 1) (layer "B.Cu") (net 8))
 (segment (start 126.454709 80.409313) (end 128.020043 80.409313) (width 1) (layer "B.Cu") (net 8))
 (segment (start 134.500647 89.145287) (end 134.500647 90.661609) (width 1) (layer "B.Cu") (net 10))
 (segment (start 134.97 88.675934) (end 134.500647 89.145287) (width 1) (layer "B.Cu") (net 10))
 (segment (start 119.537486 87.42497) (end 121.719374 87.42497) (width 1) (layer "B.Cu") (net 10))
 (segment (start 124.890274 92.981404) (end 127.018574 92.981404) (width 1) (layer "B.Cu") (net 10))
 (segment (start 118.387111 86.274595) (end 119.537486 87.42497) (width 1) (layer "B.Cu") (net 10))
 (segment (start 130.614951 94.547305) (end 134.500647 90.661609) (width 1) (layer "B.Cu") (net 10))
 (segment (start 127.018574 92.981404) (end 128.584475 94.547305) (width 1) (layer "B.Cu") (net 10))
 (segment (start 121.719374 87.42497) (end 123.454511 89.160107) (width 1) (layer "B.Cu") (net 10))
 (segment (start 123.454511 89.160107) (end 123.454511 91.545641) (width 1) (layer "B.Cu") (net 10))
 (segment (start 128.584475 94.547305) (end 130.614951 94.547305) (width 1) (layer "B.Cu") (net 10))
 (segment (start 118.387111 84.124595) (end 118.387111 86.274595) (width 1) (layer "B.Cu") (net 10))
 (segment (start 134.97 86.708709) (end 134.97 88.675934) (width 1) (layer "B.Cu") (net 10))
 (segment (start 123.454511 91.545641) (end 124.890274 92.981404) (width 1) (layer "B.Cu") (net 10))
 (segment (start 126.007111 84.124595) (end 126.007111 86.765431) (width 1) (layer "B.Cu") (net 9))
 (segment (start 132.43 87.709356) (end 132.43 86.708709) (width 1) (layer "B.Cu") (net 9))
 (segment (start 128.521389 89.279709) (end 130.859647 89.279709) (width 1) (layer "B.Cu") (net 9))
 (segment (start 126.007111 86.765431) (end 128.521389 89.279709) (width 1) (layer "B.Cu") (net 9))
 (segment (start 130.859647 89.279709) (end 132.43 87.709356) (width 1) (layer "B.Cu") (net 9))
 (segment (start 116.5 90.157616) (end 117.302327 89.355289) (width 1) (layer "B.Cu") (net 12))
 (segment (start 116.5 90.157616) (end 121.439801 90.157616) (width 1) (layer "B.Cu") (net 12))
 (segment (start 117.302327 89.355289) (end 120.183455 89.355289) (width 1) (layer "B.Cu") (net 12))
 (segment (start 120.183455 89.355289) (end 120.917442 90.089276) (width 1) (layer "B.Cu") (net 12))
 (segment (start 167.60558 72.10558) (end 168.5 73) (width 2.3) (layer "B.Cu") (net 11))
 (segment (start 162.95913 72.10558) (end 167.60558 72.10558) (width 2.3) (layer "B.Cu") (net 11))
 (segment (start 116.716045 75.329698) (end 116.716045 78.887292) (width 1) (layer "B.Cu") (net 4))
 (segment (start 116.343868 74.957521) (end 116.716045 75.329698) (width 1) (layer "B.Cu") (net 4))
 (segment (start 122.14152 82.615337) (end 122.14152 84.97397) (width 1) (layer "B.Cu") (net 4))
 (segment (start 119.763419 81.934666) (end 121.460849 81.934666) (width 1) (layer "B.Cu") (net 4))
 (segment (start 122.14152 82.615337) (end 122.14152 80.933056) (width 1) (layer "B.Cu") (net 4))
 (segment (start 121.460849 81.934666) (end 122.14152 82.615337) (width 1) (layer "B.Cu") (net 4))
 (segment (start 116.716045 78.887292) (end 119.763419 81.934666) (width 1) (layer "B.Cu") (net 4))
 (segment (start 122.14152 80.933056) (end 122.954035 80.120541) (width 1) (layer "B.Cu") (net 4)))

